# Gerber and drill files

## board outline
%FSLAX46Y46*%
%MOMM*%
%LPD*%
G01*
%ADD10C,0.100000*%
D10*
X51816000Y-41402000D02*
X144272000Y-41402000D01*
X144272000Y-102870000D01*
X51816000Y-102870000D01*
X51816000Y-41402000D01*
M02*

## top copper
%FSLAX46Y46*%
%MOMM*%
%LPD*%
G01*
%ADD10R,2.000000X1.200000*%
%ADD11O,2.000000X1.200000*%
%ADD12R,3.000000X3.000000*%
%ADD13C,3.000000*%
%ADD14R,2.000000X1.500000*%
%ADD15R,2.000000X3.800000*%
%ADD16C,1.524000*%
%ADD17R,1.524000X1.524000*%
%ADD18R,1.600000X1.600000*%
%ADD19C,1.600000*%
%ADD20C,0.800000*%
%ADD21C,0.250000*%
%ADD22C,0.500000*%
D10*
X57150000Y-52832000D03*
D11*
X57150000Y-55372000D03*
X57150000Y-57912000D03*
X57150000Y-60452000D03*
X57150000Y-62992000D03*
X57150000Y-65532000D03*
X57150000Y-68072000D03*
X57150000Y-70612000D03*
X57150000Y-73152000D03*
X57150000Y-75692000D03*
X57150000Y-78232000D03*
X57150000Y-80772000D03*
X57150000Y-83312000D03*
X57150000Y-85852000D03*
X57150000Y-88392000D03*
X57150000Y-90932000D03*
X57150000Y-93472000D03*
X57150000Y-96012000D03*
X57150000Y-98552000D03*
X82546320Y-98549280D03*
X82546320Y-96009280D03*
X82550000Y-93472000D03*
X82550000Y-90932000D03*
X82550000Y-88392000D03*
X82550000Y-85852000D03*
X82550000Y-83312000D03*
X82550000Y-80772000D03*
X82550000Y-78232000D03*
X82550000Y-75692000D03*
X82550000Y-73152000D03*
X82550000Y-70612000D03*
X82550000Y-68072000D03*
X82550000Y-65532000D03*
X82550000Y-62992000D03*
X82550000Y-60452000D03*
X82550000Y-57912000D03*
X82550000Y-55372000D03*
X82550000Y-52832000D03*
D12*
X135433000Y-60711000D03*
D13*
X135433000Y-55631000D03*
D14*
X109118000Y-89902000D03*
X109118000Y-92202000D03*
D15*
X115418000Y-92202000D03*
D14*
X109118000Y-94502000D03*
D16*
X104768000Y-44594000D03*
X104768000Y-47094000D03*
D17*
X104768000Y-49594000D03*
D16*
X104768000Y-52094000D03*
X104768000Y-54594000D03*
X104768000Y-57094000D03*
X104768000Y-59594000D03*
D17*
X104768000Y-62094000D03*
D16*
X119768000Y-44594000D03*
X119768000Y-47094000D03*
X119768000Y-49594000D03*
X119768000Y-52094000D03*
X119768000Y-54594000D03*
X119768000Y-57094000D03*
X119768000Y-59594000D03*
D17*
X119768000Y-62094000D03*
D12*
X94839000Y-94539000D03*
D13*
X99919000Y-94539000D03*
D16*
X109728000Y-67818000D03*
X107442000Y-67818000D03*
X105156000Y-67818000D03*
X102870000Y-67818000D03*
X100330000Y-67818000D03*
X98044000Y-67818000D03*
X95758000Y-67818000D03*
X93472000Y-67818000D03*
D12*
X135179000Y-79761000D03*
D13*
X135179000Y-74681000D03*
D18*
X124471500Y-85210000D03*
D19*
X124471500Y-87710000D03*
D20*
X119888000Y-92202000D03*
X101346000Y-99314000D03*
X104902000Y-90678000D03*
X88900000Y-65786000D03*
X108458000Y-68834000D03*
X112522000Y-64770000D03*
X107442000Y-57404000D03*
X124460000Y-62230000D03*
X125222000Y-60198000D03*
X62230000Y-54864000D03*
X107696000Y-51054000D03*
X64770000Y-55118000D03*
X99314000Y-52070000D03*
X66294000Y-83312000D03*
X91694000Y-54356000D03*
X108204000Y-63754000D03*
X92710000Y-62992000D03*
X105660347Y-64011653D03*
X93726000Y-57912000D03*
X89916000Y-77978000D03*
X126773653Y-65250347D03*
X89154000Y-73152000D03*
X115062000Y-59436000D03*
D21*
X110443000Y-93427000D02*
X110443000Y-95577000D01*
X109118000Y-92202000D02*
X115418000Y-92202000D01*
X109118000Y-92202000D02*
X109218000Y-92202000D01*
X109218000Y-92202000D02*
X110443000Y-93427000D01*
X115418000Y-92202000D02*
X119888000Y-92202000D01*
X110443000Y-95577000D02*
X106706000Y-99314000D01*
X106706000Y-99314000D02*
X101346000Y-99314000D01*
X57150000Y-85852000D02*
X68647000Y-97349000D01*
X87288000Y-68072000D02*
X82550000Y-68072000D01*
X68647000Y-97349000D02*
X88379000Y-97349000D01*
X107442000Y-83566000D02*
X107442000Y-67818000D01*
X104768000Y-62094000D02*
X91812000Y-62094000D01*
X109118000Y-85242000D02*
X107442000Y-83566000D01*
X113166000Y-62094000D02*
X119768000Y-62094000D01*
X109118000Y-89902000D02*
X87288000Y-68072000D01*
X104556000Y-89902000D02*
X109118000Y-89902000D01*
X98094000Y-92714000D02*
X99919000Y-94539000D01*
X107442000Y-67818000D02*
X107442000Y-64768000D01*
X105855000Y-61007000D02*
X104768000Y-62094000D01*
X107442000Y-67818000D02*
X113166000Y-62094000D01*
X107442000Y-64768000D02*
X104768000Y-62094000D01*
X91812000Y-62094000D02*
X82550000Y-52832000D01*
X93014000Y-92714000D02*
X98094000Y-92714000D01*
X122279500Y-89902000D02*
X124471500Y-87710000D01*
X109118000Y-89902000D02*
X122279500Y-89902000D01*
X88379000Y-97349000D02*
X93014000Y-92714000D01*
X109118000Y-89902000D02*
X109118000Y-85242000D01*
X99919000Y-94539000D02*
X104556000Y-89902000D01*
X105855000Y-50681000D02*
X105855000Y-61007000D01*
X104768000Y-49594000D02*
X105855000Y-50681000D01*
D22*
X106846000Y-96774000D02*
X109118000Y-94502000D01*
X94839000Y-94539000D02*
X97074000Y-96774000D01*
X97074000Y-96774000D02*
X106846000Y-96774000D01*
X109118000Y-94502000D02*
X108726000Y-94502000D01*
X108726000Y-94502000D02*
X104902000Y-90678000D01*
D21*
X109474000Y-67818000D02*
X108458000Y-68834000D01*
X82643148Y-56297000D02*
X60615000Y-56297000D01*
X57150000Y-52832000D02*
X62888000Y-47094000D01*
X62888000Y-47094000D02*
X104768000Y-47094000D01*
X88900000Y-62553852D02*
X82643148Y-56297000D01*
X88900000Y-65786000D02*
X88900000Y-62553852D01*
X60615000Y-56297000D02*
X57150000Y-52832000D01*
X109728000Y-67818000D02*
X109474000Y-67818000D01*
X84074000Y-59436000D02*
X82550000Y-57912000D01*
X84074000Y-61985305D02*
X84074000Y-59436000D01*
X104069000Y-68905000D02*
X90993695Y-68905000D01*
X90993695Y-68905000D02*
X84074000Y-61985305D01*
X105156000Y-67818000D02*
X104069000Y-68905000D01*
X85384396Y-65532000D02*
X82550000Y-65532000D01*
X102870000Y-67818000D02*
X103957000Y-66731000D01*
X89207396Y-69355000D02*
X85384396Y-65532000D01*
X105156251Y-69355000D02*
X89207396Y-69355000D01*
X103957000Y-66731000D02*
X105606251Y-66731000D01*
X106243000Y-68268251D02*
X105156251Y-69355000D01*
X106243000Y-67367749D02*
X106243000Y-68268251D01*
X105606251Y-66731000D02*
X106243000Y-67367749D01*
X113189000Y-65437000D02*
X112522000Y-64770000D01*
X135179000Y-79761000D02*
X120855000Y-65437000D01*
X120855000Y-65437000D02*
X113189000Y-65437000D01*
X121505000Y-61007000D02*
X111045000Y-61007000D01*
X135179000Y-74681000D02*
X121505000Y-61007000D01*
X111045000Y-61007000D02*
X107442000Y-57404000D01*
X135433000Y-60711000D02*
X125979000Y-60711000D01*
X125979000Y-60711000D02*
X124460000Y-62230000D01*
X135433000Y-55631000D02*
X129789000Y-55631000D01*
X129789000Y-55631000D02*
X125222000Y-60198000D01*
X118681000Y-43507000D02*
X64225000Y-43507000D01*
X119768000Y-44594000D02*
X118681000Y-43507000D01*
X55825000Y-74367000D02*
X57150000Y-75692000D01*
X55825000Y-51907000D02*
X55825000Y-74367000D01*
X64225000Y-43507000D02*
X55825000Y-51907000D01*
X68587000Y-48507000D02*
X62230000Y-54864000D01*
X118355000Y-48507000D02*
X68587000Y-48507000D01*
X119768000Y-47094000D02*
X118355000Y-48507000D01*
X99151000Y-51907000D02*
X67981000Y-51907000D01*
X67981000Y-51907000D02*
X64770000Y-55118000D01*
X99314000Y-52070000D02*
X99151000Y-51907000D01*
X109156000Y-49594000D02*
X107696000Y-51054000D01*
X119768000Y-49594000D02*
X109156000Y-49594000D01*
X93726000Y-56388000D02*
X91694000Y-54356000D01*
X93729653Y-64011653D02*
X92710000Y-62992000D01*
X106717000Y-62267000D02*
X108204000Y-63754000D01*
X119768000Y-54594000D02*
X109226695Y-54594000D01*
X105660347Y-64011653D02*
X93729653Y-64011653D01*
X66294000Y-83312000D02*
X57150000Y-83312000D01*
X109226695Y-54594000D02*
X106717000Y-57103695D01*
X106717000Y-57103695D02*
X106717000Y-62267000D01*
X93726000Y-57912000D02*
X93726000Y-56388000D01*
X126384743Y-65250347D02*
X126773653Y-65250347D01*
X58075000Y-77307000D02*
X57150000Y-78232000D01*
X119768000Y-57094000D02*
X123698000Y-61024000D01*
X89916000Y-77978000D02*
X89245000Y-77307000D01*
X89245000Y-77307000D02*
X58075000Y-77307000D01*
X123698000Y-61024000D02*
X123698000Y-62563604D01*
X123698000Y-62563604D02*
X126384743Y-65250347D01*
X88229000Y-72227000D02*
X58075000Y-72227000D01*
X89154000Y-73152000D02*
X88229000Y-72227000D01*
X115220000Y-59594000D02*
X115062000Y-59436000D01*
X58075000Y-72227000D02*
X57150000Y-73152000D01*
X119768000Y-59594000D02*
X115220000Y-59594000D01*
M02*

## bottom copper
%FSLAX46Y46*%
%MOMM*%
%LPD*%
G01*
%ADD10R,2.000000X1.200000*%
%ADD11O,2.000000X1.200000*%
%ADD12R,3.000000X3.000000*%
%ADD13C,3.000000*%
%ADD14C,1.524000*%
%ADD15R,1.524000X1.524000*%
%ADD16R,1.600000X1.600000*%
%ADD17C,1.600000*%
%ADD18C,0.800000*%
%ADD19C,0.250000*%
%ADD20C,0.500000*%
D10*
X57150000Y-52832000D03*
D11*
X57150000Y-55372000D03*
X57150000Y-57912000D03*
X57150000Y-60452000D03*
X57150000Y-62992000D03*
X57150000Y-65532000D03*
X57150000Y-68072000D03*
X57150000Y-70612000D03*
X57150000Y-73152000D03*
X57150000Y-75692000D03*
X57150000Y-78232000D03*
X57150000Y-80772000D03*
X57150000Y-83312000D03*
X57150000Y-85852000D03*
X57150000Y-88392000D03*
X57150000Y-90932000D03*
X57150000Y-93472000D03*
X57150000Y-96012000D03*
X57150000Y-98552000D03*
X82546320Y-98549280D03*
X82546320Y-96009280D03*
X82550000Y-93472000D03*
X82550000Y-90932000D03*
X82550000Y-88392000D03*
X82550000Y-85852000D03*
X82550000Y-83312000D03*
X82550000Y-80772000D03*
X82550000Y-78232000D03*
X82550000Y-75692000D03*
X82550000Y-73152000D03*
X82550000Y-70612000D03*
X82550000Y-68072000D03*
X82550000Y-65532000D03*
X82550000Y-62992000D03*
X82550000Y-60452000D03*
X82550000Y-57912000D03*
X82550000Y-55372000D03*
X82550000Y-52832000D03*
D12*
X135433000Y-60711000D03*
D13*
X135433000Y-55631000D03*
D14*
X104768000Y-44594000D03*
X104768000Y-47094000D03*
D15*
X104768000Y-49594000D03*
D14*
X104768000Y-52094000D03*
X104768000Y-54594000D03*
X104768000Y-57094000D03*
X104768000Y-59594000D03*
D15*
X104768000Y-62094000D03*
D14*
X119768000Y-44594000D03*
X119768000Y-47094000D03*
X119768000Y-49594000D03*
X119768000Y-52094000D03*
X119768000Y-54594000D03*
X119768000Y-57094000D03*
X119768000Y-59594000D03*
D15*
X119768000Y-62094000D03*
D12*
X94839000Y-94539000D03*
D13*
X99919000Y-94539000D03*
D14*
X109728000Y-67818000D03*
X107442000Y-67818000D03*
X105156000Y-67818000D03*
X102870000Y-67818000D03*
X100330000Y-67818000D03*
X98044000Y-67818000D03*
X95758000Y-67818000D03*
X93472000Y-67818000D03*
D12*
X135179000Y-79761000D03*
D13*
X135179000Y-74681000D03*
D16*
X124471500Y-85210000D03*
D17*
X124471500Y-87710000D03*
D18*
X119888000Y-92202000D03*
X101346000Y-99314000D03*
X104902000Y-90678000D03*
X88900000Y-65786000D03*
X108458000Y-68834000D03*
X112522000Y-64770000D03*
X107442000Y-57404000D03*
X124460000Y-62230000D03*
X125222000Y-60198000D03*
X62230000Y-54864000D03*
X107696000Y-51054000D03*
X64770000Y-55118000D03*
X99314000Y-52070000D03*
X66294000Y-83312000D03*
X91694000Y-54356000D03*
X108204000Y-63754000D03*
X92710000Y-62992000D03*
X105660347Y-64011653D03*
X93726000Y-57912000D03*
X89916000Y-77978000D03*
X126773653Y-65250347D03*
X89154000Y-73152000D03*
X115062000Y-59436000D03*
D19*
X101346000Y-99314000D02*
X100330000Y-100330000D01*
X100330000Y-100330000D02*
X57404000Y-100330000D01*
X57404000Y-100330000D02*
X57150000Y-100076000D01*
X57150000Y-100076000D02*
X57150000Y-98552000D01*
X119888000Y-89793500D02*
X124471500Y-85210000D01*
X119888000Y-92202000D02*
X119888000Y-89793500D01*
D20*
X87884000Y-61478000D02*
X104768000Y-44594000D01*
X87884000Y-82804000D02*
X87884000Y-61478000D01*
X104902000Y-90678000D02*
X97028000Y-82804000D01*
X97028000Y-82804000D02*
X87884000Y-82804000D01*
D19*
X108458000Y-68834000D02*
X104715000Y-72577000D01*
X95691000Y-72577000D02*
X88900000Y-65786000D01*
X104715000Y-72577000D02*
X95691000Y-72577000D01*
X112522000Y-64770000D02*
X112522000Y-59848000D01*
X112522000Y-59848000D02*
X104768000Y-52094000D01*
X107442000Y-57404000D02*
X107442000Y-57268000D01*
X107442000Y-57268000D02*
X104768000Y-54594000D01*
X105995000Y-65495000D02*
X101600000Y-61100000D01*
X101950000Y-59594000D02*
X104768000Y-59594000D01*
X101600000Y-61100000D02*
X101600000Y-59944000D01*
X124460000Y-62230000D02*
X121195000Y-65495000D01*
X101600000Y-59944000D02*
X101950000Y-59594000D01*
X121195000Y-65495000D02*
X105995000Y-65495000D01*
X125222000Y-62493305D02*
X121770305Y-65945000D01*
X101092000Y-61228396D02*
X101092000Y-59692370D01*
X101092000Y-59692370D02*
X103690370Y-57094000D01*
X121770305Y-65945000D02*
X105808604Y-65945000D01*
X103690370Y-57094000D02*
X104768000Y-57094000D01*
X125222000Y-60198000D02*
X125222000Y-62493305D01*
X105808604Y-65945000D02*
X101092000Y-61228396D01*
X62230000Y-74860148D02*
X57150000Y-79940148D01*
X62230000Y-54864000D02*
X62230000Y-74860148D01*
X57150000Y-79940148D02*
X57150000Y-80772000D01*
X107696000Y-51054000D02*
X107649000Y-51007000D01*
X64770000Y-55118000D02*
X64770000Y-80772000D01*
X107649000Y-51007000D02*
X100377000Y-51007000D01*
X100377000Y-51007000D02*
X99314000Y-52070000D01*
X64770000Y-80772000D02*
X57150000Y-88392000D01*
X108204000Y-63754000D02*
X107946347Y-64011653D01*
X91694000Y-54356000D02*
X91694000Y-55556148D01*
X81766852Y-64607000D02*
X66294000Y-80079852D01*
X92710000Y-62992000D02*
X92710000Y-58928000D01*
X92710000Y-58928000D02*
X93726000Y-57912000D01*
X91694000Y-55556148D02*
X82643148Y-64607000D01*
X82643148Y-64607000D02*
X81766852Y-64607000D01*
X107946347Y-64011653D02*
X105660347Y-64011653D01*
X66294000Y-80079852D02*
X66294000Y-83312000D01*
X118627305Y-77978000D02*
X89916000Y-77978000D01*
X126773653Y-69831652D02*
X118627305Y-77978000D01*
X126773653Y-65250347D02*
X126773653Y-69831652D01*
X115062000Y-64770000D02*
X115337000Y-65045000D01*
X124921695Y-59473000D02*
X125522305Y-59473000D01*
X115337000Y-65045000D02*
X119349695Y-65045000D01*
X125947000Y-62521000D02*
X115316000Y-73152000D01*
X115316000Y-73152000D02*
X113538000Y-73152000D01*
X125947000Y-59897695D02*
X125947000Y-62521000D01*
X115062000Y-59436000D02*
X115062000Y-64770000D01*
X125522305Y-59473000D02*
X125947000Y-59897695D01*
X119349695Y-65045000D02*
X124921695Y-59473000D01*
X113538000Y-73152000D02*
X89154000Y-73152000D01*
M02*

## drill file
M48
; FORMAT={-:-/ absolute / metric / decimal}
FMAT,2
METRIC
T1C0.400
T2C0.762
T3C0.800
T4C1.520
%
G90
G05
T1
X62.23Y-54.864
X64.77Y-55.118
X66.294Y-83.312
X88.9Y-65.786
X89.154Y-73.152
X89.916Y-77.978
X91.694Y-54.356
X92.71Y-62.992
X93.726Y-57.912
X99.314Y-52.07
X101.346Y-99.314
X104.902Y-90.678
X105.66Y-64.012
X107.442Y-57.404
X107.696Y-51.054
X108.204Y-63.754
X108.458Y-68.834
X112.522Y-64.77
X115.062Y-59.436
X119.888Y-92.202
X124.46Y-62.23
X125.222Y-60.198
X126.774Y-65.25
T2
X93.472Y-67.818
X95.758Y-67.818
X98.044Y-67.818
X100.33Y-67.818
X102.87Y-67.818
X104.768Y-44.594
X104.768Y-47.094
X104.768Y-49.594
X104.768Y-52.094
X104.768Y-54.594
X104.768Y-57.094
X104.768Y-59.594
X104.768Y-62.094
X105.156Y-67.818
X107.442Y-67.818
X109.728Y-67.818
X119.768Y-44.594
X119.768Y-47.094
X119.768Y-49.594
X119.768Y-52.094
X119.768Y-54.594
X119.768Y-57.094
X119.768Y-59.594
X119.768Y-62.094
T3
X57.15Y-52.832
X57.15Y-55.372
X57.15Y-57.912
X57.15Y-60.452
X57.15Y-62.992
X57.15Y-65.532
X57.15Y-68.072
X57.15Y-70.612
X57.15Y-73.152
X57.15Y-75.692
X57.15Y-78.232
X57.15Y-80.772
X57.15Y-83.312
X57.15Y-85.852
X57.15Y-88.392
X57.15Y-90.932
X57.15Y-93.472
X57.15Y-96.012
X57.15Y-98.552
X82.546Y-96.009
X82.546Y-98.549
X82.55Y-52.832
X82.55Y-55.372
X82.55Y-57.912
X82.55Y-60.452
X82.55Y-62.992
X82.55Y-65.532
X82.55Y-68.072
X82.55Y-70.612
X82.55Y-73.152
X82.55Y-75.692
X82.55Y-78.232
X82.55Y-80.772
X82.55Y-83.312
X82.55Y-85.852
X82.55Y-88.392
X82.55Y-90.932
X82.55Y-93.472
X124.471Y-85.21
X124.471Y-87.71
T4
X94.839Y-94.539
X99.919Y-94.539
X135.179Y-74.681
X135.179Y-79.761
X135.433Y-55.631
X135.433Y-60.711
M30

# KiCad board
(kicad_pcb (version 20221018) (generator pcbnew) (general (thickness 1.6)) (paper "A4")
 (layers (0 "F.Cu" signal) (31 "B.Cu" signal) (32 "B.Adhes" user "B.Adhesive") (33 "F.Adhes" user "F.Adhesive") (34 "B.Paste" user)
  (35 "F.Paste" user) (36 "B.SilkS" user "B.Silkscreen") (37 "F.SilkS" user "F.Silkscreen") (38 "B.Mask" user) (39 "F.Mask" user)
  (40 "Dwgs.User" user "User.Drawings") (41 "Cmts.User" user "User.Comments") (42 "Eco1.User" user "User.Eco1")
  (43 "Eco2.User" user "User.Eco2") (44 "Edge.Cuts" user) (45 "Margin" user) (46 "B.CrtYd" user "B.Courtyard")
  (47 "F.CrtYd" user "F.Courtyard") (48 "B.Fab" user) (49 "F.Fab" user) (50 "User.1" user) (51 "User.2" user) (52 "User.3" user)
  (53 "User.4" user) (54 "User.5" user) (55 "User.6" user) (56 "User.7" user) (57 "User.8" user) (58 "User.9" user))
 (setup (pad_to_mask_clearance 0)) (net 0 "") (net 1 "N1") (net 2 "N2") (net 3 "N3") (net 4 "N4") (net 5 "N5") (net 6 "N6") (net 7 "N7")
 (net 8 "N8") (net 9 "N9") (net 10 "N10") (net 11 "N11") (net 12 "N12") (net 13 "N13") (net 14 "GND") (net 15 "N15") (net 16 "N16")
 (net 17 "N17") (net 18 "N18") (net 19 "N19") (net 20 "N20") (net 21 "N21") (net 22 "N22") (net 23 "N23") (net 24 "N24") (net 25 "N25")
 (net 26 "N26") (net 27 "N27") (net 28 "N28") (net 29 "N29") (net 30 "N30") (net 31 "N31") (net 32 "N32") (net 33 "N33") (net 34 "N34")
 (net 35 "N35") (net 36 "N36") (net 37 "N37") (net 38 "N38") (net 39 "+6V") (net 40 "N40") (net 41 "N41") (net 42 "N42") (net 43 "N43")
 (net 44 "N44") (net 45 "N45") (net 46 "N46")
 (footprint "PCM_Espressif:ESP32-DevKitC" (layer "F.Cu") (at 57.15 52.832)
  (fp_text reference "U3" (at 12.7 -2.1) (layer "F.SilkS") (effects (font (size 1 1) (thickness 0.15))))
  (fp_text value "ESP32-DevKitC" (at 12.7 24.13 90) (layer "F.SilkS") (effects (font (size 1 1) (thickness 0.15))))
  (pad "1" thru_hole rect (at 0 0 270) (size 1.2 2) (drill 0.8) (layers "*.Cu" "*.Mask") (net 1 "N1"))
  (pad "2" thru_hole oval (at 0 2.54 270) (size 1.2 2) (drill 0.8) (layers "*.Cu" "*.Mask") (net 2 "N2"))
  (pad "3" thru_hole oval (at 0 5.08 270) (size 1.2 2) (drill 0.8) (layers "*.Cu" "*.Mask") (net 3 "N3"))
  (pad "4" thru_hole oval (at 0 7.62 270) (size 1.2 2) (drill 0.8) (layers "*.Cu" "*.Mask") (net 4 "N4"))
  (pad "5" thru_hole oval (at 0 10.16 270) (size 1.2 2) (drill 0.8) (layers "*.Cu" "*.Mask") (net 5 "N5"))
  (pad "6" thru_hole oval (at 0 12.7 270) (size 1.2 2) (drill 0.8) (layers "*.Cu" "*.Mask") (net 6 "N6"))
  (pad "7" thru_hole oval (at 0 15.24 270) (size 1.2 2) (drill 0.8) (layers "*.Cu" "*.Mask") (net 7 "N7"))
  (pad "8" thru_hole oval (at 0 17.78 270) (size 1.2 2) (drill 0.8) (layers "*.Cu" "*.Mask") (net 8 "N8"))
  (pad "9" thru_hole oval (at 0 20.32 270) (size 1.2 2) (drill 0.8) (layers "*.Cu" "*.Mask") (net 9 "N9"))
  (pad "10" thru_hole oval (at 0 22.86 270) (size 1.2 2) (drill 0.8) (layers "*.Cu" "*.Mask") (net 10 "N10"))
  (pad "11" thru_hole oval (at 0 25.4 270) (size 1.2 2) (drill 0.8) (layers "*.Cu" "*.Mask") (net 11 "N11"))
  (pad "12" thru_hole oval (at 0 27.94 270) (size 1.2 2) (drill 0.8) (layers "*.Cu" "*.Mask") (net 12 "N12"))
  (pad "13" thru_hole oval (at 0 30.48 270) (size 1.2 2) (drill 0.8) (layers "*.Cu" "*.Mask") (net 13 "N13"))
  (pad "14" thru_hole oval (at 0 33.02 270) (size 1.2 2) (drill 0.8) (layers "*.Cu" "*.Mask") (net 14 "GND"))
  (pad "15" thru_hole oval (at 0 35.56 270) (size 1.2 2) (drill 0.8) (layers "*.Cu" "*.Mask") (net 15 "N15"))
  (pad "16" thru_hole oval (at 0 38.1 270) (size 1.2 2) (drill 0.8) (layers "*.Cu" "*.Mask") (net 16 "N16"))
  (pad "17" thru_hole oval (at 0 40.64 270) (size 1.2 2) (drill 0.8) (layers "*.Cu" "*.Mask") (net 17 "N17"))
  (pad "18" thru_hole oval (at 0 43.18 270) (size 1.2 2) (drill 0.8) (layers "*.Cu" "*.Mask") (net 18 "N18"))
  (pad "19" thru_hole oval (at 0 45.72 270) (size 1.2 2) (drill 0.8) (layers "*.Cu" "*.Mask") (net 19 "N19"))
  (pad "20" thru_hole oval (at 25.39632 45.71728 270) (size 1.2 2) (drill 0.8) (layers "*.Cu" "*.Mask") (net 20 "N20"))
  (pad "21" thru_hole oval (at 25.39632 43.17728 270) (size 1.2 2) (drill 0.8) (layers "*.Cu" "*.Mask") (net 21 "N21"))
  (pad "22" thru_hole oval (at 25.4 40.64 270) (size 1.2 2) (drill 0.8) (layers "*.Cu" "*.Mask") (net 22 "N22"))
  (pad "23" thru_hole oval (at 25.4 38.1 270) (size 1.2 2) (drill 0.8) (layers "*.Cu" "*.Mask") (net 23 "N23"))
  (pad "24" thru_hole oval (at 25.4 35.56 270) (size 1.2 2) (drill 0.8) (layers "*.Cu" "*.Mask") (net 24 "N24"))
  (pad "25" thru_hole oval (at 25.4 33.02 270) (size 1.2 2) (drill 0.8) (layers "*.Cu" "*.Mask") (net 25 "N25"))
  (pad "26" thru_hole oval (at 25.4 30.48 270) (size 1.2 2) (drill 0.8) (layers "*.Cu" "*.Mask") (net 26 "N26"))
  (pad "27" thru_hole oval (at 25.4 27.94 270) (size 1.2 2) (drill 0.8) (layers "*.Cu" "*.Mask") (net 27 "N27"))
  (pad "28" thru_hole oval (at 25.4 25.4 270) (size 1.2 2) (drill 0.8) (layers "*.Cu" "*.Mask") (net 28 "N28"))
  (pad "29" thru_hole oval (at 25.4 22.86 270) (size 1.2 2) (drill 0.8) (layers "*.Cu" "*.Mask") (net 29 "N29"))
  (pad "30" thru_hole oval (at 25.4 20.32 270) (size 1.2 2) (drill 0.8) (layers "*.Cu" "*.Mask") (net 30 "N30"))
  (pad "31" thru_hole oval (at 25.4 17.78 270) (size 1.2 2) (drill 0.8) (layers "*.Cu" "*.Mask") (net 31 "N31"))
  (pad "32" thru_hole oval (at 25.4 15.24 270) (size 1.2 2) (drill 0.8) (layers "*.Cu" "*.Mask") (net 14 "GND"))
  (pad "33" thru_hole oval (at 25.4 12.7 270) (size 1.2 2) (drill 0.8) (layers "*.Cu" "*.Mask") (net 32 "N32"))
  (pad "34" thru_hole oval (at 25.4 10.16 270) (size 1.2 2) (drill 0.8) (layers "*.Cu" "*.Mask") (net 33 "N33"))
  (pad "35" thru_hole oval (at 25.4 7.62 270) (size 1.2 2) (drill 0.8) (layers "*.Cu" "*.Mask") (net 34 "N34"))
  (pad "36" thru_hole oval (at 25.4 5.08 270) (size 1.2 2) (drill 0.8) (layers "*.Cu" "*.Mask") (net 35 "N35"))
  (pad "37" thru_hole oval (at 25.4 2.54 270) (size 1.2 2) (drill 0.8) (layers "*.Cu" "*.Mask") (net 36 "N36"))
  (pad "38" thru_hole oval (at 25.4 0 270) (size 1.2 2) (drill 0.8) (layers "*.Cu" "*.Mask") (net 14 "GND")))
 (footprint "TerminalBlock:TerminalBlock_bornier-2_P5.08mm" (layer "F.Cu") (at 135.433 60.711 90)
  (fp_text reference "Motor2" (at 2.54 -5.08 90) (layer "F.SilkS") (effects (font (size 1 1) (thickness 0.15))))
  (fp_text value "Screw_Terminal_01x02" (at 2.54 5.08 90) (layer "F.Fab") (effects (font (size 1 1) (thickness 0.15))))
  (pad "1" thru_hole rect (at 0 0 90) (size 3 3) (drill 1.52) (layers "*.Cu" "*.Mask") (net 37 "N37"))
  (pad "2" thru_hole circle (at 5.08 0 90) (size 3 3) (drill 1.52) (layers "*.Cu" "*.Mask") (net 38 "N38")))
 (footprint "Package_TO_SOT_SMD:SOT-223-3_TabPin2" (layer "F.Cu") (at 112.268 92.202)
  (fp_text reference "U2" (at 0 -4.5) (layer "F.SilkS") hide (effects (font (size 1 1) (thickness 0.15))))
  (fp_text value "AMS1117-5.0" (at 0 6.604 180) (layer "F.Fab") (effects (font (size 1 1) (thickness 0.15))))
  (pad "1" smd rect (at -3.15 -2.3) (size 2 1.5) (layers "F.Cu" "F.Paste" "F.Mask") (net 14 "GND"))
  (pad "2" smd rect (at -3.15 0) (size 2 1.5) (layers "F.Cu" "F.Paste" "F.Mask") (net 19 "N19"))
  (pad "2" smd rect (at 3.15 0) (size 2 3.8) (layers "F.Cu" "F.Paste" "F.Mask") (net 19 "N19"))
  (pad "3" smd rect (at -3.15 2.3) (size 2 1.5) (layers "F.Cu" "F.Paste" "F.Mask") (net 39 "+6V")))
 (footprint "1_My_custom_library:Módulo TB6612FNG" (layer "F.Cu") (at 112.268 53.594)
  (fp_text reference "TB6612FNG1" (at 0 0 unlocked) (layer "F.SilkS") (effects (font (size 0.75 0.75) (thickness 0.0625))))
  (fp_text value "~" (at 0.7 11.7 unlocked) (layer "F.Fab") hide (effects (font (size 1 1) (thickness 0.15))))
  (pad "1" thru_hole circle (at -7.5 -9) (size 1.524 1.524) (drill 0.762) (layers "*.Cu" "*.Mask") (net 39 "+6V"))
  (pad "2" thru_hole circle (at -7.5 -6.5) (size 1.524 1.524) (drill 0.762) (layers "*.Cu" "*.Mask") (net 1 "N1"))
  (pad "3" thru_hole rect (at -7.5 -4) (size 1.524 1.524) (drill 0.762) (layers "*.Cu" "*.Mask") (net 14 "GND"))
  (pad "4" thru_hole circle (at -7.5 -1.5) (size 1.524 1.524) (drill 0.762) (layers "*.Cu" "*.Mask") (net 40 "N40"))
  (pad "5" thru_hole circle (at -7.5 1) (size 1.524 1.524) (drill 0.762) (layers "*.Cu" "*.Mask") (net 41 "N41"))
  (pad "6" thru_hole circle (at -7.5 3.5) (size 1.524 1.524) (drill 0.762) (layers "*.Cu" "*.Mask") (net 38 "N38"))
  (pad "7" thru_hole circle (at -7.5 6) (size 1.524 1.524) (drill 0.762) (layers "*.Cu" "*.Mask") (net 37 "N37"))
  (pad "8" thru_hole rect (at -7.5 8.5) (size 1.524 1.524) (drill 0.762) (layers "*.Cu" "*.Mask") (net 14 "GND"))
  (pad "9" thru_hole circle (at 7.5 -9) (size 1.524 1.524) (drill 0.762) (layers "*.Cu" "*.Mask") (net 10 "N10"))
  (pad "10" thru_hole circle (at 7.5 -6.5) (size 1.524 1.524) (drill 0.762) (layers "*.Cu" "*.Mask") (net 12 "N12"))
  (pad "11" thru_hole circle (at 7.5 -4) (size 1.524 1.524) (drill 0.762) (layers "*.Cu" "*.Mask") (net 15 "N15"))
  (pad "12" thru_hole circle (at 7.5 -1.5) (size 1.524 1.524) (drill 0.762) (layers "*.Cu" "*.Mask") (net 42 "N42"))
  (pad "13" thru_hole circle (at 7.5 1) (size 1.524 1.524) (drill 0.762) (layers "*.Cu" "*.Mask") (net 13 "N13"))
  (pad "14" thru_hole circle (at 7.5 3.5) (size 1.524 1.524) (drill 0.762) (layers "*.Cu" "*.Mask") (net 11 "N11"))
  (pad "15" thru_hole circle (at 7.5 6) (size 1.524 1.524) (drill 0.762) (layers "*.Cu" "*.Mask") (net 9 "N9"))
  (pad "16" thru_hole rect (at 7.5 8.5) (size 1.524 1.524) (drill 0.762) (layers "*.Cu" "*.Mask") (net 14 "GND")))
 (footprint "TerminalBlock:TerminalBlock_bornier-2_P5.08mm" (layer "F.Cu") (at 94.839 94.539)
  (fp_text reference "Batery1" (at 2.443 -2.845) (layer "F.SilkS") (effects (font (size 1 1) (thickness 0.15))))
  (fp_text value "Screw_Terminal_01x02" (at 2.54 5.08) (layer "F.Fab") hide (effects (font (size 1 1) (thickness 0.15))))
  (pad "1" thru_hole rect (at 0 0) (size 3 3) (drill 1.52) (layers "*.Cu" "*.Mask") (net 39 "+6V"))
  (pad "2" thru_hole circle (at 5.08 0) (size 3 3) (drill 1.52) (layers "*.Cu" "*.Mask") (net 14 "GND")))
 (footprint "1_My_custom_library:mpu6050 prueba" (layer "F.Cu") (at 101.346 73.406 -90)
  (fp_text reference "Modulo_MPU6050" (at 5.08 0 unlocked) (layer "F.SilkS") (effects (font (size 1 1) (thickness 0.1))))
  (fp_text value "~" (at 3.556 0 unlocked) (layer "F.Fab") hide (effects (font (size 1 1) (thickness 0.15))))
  (pad "1" thru_hole circle (at -5.588 -8.382 270) (size 1.524 1.524) (drill 0.762) (layers "*.Cu" "*.Mask") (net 1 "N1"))
  (pad "2" thru_hole circle (at -5.588 -6.096 270) (size 1.524 1.524) (drill 0.762) (layers "*.Cu" "*.Mask") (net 14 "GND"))
  (pad "3" thru_hole circle (at -5.588 -3.81 270) (size 1.524 1.524) (drill 0.762) (layers "*.Cu" "*.Mask") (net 35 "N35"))
  (pad "4" thru_hole circle (at -5.588 -1.524 270) (size 1.524 1.524) (drill 0.762) (layers "*.Cu" "*.Mask") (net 32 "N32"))
  (pad "5" thru_hole circle (at -5.588 1.016 270) (size 1.524 1.524) (drill 0.762) (layers "*.Cu" "*.Mask") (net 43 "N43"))
  (pad "6" thru_hole circle (at -5.588 3.302 270) (size 1.524 1.524) (drill 0.762) (layers "*.Cu" "*.Mask") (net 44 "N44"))
  (pad "7" thru_hole circle (at -5.588 5.588 270) (size 1.524 1.524) (drill 0.762) (layers "*.Cu" "*.Mask") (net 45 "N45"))
  (pad "8" thru_hole circle (at -5.588 7.874 270) (size 1.524 1.524) (drill 0.762) (layers "*.Cu" "*.Mask") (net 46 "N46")))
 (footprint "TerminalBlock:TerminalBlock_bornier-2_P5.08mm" (layer "F.Cu") (at 135.179 79.761 90)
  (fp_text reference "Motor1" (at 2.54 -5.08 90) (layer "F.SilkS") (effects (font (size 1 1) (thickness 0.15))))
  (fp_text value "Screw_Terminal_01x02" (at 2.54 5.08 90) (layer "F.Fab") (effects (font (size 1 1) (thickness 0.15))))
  (pad "1" thru_hole rect (at 0 0 90) (size 3 3) (drill 1.52) (layers "*.Cu" "*.Mask") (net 40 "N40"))
  (pad "2" thru_hole circle (at 5.08 0 90) (size 3 3) (drill 1.52) (layers "*.Cu" "*.Mask") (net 41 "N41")))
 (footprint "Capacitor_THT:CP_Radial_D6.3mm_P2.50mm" (layer "F.Cu") (at 124.4715 85.21 -90)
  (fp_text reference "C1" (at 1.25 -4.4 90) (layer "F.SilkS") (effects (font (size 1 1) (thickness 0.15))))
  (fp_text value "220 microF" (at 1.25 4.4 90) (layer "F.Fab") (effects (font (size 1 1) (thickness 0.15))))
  (pad "1" thru_hole rect (at 0 0 270) (size 1.6 1.6) (drill 0.8) (layers "*.Cu" "*.Mask") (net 19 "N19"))
  (pad "2" thru_hole circle (at 2.5 0 270) (size 1.6 1.6) (drill 0.8) (layers "*.Cu" "*.Mask") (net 14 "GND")))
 (gr_rect (start 51.816 41.402) (end 144.272 102.87) (stroke (width 0.1) (type default)) (fill none) (layer "Edge.Cuts"))
 (segment (start 110.443 93.427) (end 110.443 95.577) (width 0.25) (layer "F.Cu") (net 19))
 (segment (start 109.118 92.202) (end 115.418 92.202) (width 0.25) (layer "F.Cu") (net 19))
 (segment (start 109.118 92.202) (end 109.218 92.202) (width 0.25) (layer "F.Cu") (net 19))
 (segment (start 109.218 92.202) (end 110.443 93.427) (width 0.25) (layer "F.Cu") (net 19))
 (segment (start 115.418 92.202) (end 119.888 92.202) (width 0.25) (layer "F.Cu") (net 19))
 (segment (start 110.443 95.577) (end 106.706 99.314) (width 0.25) (layer "F.Cu") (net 19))
 (segment (start 106.706 99.314) (end 101.346 99.314) (width 0.25) (layer "F.Cu") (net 19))
 (via (at 119.888 92.202) (size 0.8) (drill 0.4) (layers "F.Cu" "B.Cu") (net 19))
 (via (at 101.346 99.314) (size 0.8) (drill 0.4) (layers "F.Cu" "B.Cu") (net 19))
 (segment (start 101.346 99.314) (end 100.33 100.33) (width 0.25) (layer "B.Cu") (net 19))
 (segment (start 100.33 100.33) (end 57.404 100.33) (width 0.25) (layer "B.Cu") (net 19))
 (segment (start 57.404 100.33) (end 57.15 100.076) (width 0.25) (layer "B.Cu") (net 19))
 (segment (start 57.15 100.076) (end 57.15 98.552) (width 0.25) (layer "B.Cu") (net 19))
 (segment (start 119.888 89.7935) (end 124.4715 85.21) (width 0.25) (layer "B.Cu") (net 19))
 (segment (start 119.888 92.202) (end 119.888 89.7935) (width 0.25) (layer "B.Cu") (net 19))
 (segment (start 57.15 85.852) (end 68.647 97.349) (width 0.25) (layer "F.Cu") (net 14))
 (segment (start 87.288 68.072) (end 82.55 68.072) (width 0.25) (layer "F.Cu") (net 14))
 (segment (start 68.647 97.349) (end 88.379 97.349) (width 0.25) (layer "F.Cu") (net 14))
 (segment (start 107.442 83.566) (end 107.442 67.818) (width 0.25) (layer "F.Cu") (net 14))
 (segment (start 104.768 62.094) (end 91.812 62.094) (width 0.25) (layer "F.Cu") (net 14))
 (segment (start 109.118 85.242) (end 107.442 83.566) (width 0.25) (layer "F.Cu") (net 14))
 (segment (start 113.166 62.094) (end 119.768 62.094) (width 0.25) (layer "F.Cu") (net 14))
 (segment (start 109.118 89.902) (end 87.288 68.072) (width 0.25) (layer "F.Cu") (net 14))
 (segment (start 104.556 89.902) (end 109.118 89.902) (width 0.25) (layer "F.Cu") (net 14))
 (segment (start 98.094 92.714) (end 99.919 94.539) (width 0.25) (layer "F.Cu") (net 14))
 (segment (start 107.442 67.818) (end 107.442 64.768) (width 0.25) (layer "F.Cu") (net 14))
 (segment (start 105.855 61.007) (end 104.768 62.094) (width 0.25) (layer "F.Cu") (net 14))
 (segment (start 107.442 67.818) (end 113.166 62.094) (width 0.25) (layer "F.Cu") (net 14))
 (segment (start 107.442 64.768) (end 104.768 62.094) (width 0.25) (layer "F.Cu") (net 14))
 (segment (start 91.812 62.094) (end 82.55 52.832) (width 0.25) (layer "F.Cu") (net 14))
 (segment (start 93.014 92.714) (end 98.094 92.714) (width 0.25) (layer "F.Cu") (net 14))
 (segment (start 122.2795 89.902) (end 124.4715 87.71) (width 0.25) (layer "F.Cu") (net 14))
 (segment (start 109.118 89.902) (end 122.2795 89.902) (width 0.25) (layer "F.Cu") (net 14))
 (segment (start 88.379 97.349) (end 93.014 92.714) (width 0.25) (layer "F.Cu") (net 14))
 (segment (start 109.118 89.902) (end 109.118 85.242) (width 0.25) (layer "F.Cu") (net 14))
 (segment (start 99.919 94.539) (end 104.556 89.902) (width 0.25) (layer "F.Cu") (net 14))
 (segment (start 105.855 50.681) (end 105.855 61.007) (width 0.25) (layer "F.Cu") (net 14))
 (segment (start 104.768 49.594) (end 105.855 50.681) (width 0.25) (layer "F.Cu") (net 14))
 (segment (start 106.846 96.774) (end 109.118 94.502) (width 0.5) (layer "F.Cu") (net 39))
 (segment (start 94.839 94.539) (end 97.074 96.774) (width 0.5) (layer "F.Cu") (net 39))
 (segment (start 97.074 96.774) (end 106.846 96.774) (width 0.5) (layer "F.Cu") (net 39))
 (segment (start 109.118 94.502) (end 108.726 94.502) (width 0.5) (layer "F.Cu") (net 39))
 (segment (start 108.726 94.502) (end 104.902 90.678) (width 0.5) (layer "F.Cu") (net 39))
 (via (at 104.902 90.678) (size 0.8) (drill 0.4) (layers "F.Cu" "B.Cu") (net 39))
 (segment (start 87.884 61.478) (end 104.768 44.594) (width 0.5) (layer "B.Cu") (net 39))
 (segment (start 87.884 82.804) (end 87.884 61.478) (width 0.5) (layer "B.Cu") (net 39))
 (segment (start 104.902 90.678) (end 97.028 82.804) (width 0.5) (layer "B.Cu") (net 39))
 (segment (start 97.028 82.804) (end 87.884 82.804) (width 0.5) (layer "B.Cu") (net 39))
 (segment (start 109.474 67.818) (end 108.458 68.834) (width 0.25) (layer "F.Cu") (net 1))
 (segment (start 82.643148 56.297) (end 60.615 56.297) (width 0.25) (layer "F.Cu") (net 1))
 (segment (start 57.15 52.832) (end 62.888 47.094) (width 0.25) (layer "F.Cu") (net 1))
 (segment (start 62.888 47.094) (end 104.768 47.094) (width 0.25) (layer "F.Cu") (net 1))
 (segment (start 88.9 62.553852) (end 82.643148 56.297) (width 0.25) (layer "F.Cu") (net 1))
 (segment (start 88.9 65.786) (end 88.9 62.553852) (width 0.25) (layer "F.Cu") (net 1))
 (segment (start 60.615 56.297) (end 57.15 52.832) (width 0.25) (layer "F.Cu") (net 1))
 (segment (start 109.728 67.818) (end 109.474 67.818) (width 0.25) (layer "F.Cu") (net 1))
 (via (at 88.9 65.786) (size 0.8) (drill 0.4) (layers "F.Cu" "B.Cu") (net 1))
 (via (at 108.458 68.834) (size 0.8) (drill 0.4) (layers "F.Cu" "B.Cu") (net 1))
 (segment (start 108.458 68.834) (end 104.715 72.577) (width 0.25) (layer "B.Cu") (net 1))
 (segment (start 95.691 72.577) (end 88.9 65.786) (width 0.25) (layer "B.Cu") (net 1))
 (segment (start 104.715 72.577) (end 95.691 72.577) (width 0.25) (layer "B.Cu") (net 1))
 (segment (start 84.074 59.436) (end 82.55 57.912) (width 0.25) (layer "F.Cu") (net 35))
 (segment (start 84.074 61.985305) (end 84.074 59.436) (width 0.25) (layer "F.Cu") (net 35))
 (segment (start 104.069 68.905) (end 90.993695 68.905) (width 0.25) (layer "F.Cu") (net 35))
 (segment (start 90.993695 68.905) (end 84.074 61.985305) (width 0.25) (layer "F.Cu") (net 35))
 (segment (start 105.156 67.818) (end 104.069 68.905) (width 0.25) (layer "F.Cu") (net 35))
 (segment (start 85.384396 65.532) (end 82.55 65.532) (width 0.25) (layer "F.Cu") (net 32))
 (segment (start 102.87 67.818) (end 103.957 66.731) (width 0.25) (layer "F.Cu") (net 32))
 (segment (start 89.207396 69.355) (end 85.384396 65.532) (width 0.25) (layer "F.Cu") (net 32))
 (segment (start 105.156251 69.355) (end 89.207396 69.355) (width 0.25) (layer "F.Cu") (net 32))
 (segment (start 103.957 66.731) (end 105.606251 66.731) (width 0.25) (layer "F.Cu") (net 32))
 (segment (start 106.243 68.268251) (end 105.156251 69.355) (width 0.25) (layer "F.Cu") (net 32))
 (segment (start 106.243 67.367749) (end 106.243 68.268251) (width 0.25) (layer "F.Cu") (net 32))
 (segment (start 105.606251 66.731) (end 106.243 67.367749) (width 0.25) (layer "F.Cu") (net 32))
 (segment (start 113.189 65.437) (end 112.522 64.77) (width 0.25) (layer "F.Cu") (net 40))
 (segment (start 135.179 79.761) (end 120.855 65.437) (width 0.25) (layer "F.Cu") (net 40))
 (segment (start 120.855 65.437) (end 113.189 65.437) (width 0.25) (layer "F.Cu") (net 40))
 (via (at 112.522 64.77) (size 0.8) (drill 0.4) (layers "F.Cu" "B.Cu") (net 40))
 (segment (start 112.522 64.77) (end 112.522 59.848) (width 0.25) (layer "B.Cu") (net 40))
 (segment (start 112.522 59.848) (end 104.768 52.094) (width 0.25) (layer "B.Cu") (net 40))
 (segment (start 121.505 61.007) (end 111.045 61.007) (width 0.25) (layer "F.Cu") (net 41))
 (segment (start 135.179 74.681) (end 121.505 61.007) (width 0.25) (layer "F.Cu") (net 41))
 (segment (start 111.045 61.007) (end 107.442 57.404) (width 0.25) (layer "F.Cu") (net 41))
 (via (at 107.442 57.404) (size 0.8) (drill 0.4) (layers "F.Cu" "B.Cu") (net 41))
 (segment (start 107.442 57.404) (end 107.442 57.268) (width 0.25) (layer "B.Cu") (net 41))
 (segment (start 107.442 57.268) (end 104.768 54.594) (width 0.25) (layer "B.Cu") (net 41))
 (segment (start 135.433 60.711) (end 125.979 60.711) (width 0.25) (layer "F.Cu") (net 37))
 (segment (start 125.979 60.711) (end 124.46 62.23) (width 0.25) (layer "F.Cu") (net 37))
 (via (at 124.46 62.23) (size 0.8) (drill 0.4) (layers "F.Cu" "B.Cu") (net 37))
 (segment (start 105.995 65.495) (end 101.6 61.1) (width 0.25) (layer "B.Cu") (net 37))
 (segment (start 101.95 59.594) (end 104.768 59.594) (width 0.25) (layer "B.Cu") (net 37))
 (segment (start 101.6 61.1) (end 101.6 59.944) (width 0.25) (layer "B.Cu") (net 37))
 (segment (start 124.46 62.23) (end 121.195 65.495) (width 0.25) (layer "B.Cu") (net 37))
 (segment (start 101.6 59.944) (end 101.95 59.594) (width 0.25) (layer "B.Cu") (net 37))
 (segment (start 121.195 65.495) (end 105.995 65.495) (width 0.25) (layer "B.Cu") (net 37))
 (segment (start 135.433 55.631) (end 129.789 55.631) (width 0.25) (layer "F.Cu") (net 38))
 (segment (start 129.789 55.631) (end 125.222 60.198) (width 0.25) (layer "F.Cu") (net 38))
 (via (at 125.222 60.198) (size 0.8) (drill 0.4) (layers "F.Cu" "B.Cu") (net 38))
 (segment (start 125.222 62.493305) (end 121.770305 65.945) (width 0.25) (layer "B.Cu") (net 38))
 (segment (start 101.092 61.228396) (end 101.092 59.69237) (width 0.25) (layer "B.Cu") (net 38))
 (segment (start 101.092 59.69237) (end 103.69037 57.094) (width 0.25) (layer "B.Cu") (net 38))
 (segment (start 121.770305 65.945) (end 105.808604 65.945) (width 0.25) (layer "B.Cu") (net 38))
 (segment (start 103.69037 57.094) (end 104.768 57.094) (width 0.25) (layer "B.Cu") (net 38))
 (segment (start 125.222 60.198) (end 125.222 62.493305) (width 0.25) (layer "B.Cu") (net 38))
 (segment (start 105.808604 65.945) (end 101.092 61.228396) (width 0.25) (layer "B.Cu") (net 38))
 (segment (start 118.681 43.507) (end 64.225 43.507) (width 0.25) (layer "F.Cu") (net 10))
 (segment (start 119.768 44.594) (end 118.681 43.507) (width 0.25) (layer "F.Cu") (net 10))
 (segment (start 55.825 74.367) (end 57.15 75.692) (width 0.25) (layer "F.Cu") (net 10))
 (segment (start 55.825 51.907) (end 55.825 74.367) (width 0.25) (layer "F.Cu") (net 10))
 (segment (start 64.225 43.507) (end 55.825 51.907) (width 0.25) (layer "F.Cu") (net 10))
 (segment (start 68.587 48.507) (end 62.23 54.864) (width 0.25) (layer "F.Cu") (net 12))
 (segment (start 118.355 48.507) (end 68.587 48.507) (width 0.25) (layer "F.Cu") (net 12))
 (segment (start 119.768 47.094) (end 118.355 48.507) (width 0.25) (layer "F.Cu") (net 12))
 (via (at 62.23 54.864) (size 0.8) (drill 0.4) (layers "F.Cu" "B.Cu") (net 12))
 (segment (start 62.23 74.860148) (end 57.15 79.940148) (width 0.25) (layer "B.Cu") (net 12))
 (segment (start 62.23 54.864) (end 62.23 74.860148) (width 0.25) (layer "B.Cu") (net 12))
 (segment (start 57.15 79.940148) (end 57.15 80.772) (width 0.25) (layer "B.Cu") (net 12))
 (segment (start 99.151 51.907) (end 67.981 51.907) (width 0.25) (layer "F.Cu") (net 15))
 (segment (start 67.981 51.907) (end 64.77 55.118) (width 0.25) (layer "F.Cu") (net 15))
 (segment (start 99.314 52.07) (end 99.151 51.907) (width 0.25) (layer "F.Cu") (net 15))
 (segment (start 109.156 49.594) (end 107.696 51.054) (width 0.25) (layer "F.Cu") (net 15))
 (segment (start 119.768 49.594) (end 109.156 49.594) (width 0.25) (layer "F.Cu") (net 15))
 (via (at 107.696 51.054) (size 0.8) (drill 0.4) (layers "F.Cu" "B.Cu") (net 15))
 (via (at 64.77 55.118) (size 0.8) (drill 0.4) (layers "F.Cu" "B.Cu") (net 15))
 (via (at 99.314 52.07) (size 0.8) (drill 0.4) (layers "F.Cu" "B.Cu") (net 15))
 (segment (start 107.696 51.054) (end 107.649 51.007) (width 0.25) (layer "B.Cu") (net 15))
 (segment (start 64.77 55.118) (end 64.77 80.772) (width 0.25) (layer "B.Cu") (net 15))
 (segment (start 107.649 51.007) (end 100.377 51.007) (width 0.25) (layer "B.Cu") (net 15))
 (segment (start 100.377 51.007) (end 99.314 52.07) (width 0.25) (layer "B.Cu") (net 15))
 (segment (start 64.77 80.772) (end 57.15 88.392) (width 0.25) (layer "B.Cu") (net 15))
 (segment (start 93.726 56.388) (end 91.694 54.356) (width 0.25) (layer "F.Cu") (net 13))
 (segment (start 93.729653 64.011653) (end 92.71 62.992) (width 0.25) (layer "F.Cu") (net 13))
 (segment (start 106.717 62.267) (end 108.204 63.754) (width 0.25) (layer "F.Cu") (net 13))
 (segment (start 119.768 54.594) (end 109.226695 54.594) (width 0.25) (layer "F.Cu") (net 13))
 (segment (start 105.660347 64.011653) (end 93.729653 64.011653) (width 0.25) (layer "F.Cu") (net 13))
 (segment (start 66.294 83.312) (end 57.15 83.312) (width 0.25) (layer "F.Cu") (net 13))
 (segment (start 109.226695 54.594) (end 106.717 57.103695) (width 0.25) (layer "F.Cu") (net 13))
 (segment (start 106.717 57.103695) (end 106.717 62.267) (width 0.25) (layer "F.Cu") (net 13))
 (segment (start 93.726 57.912) (end 93.726 56.388) (width 0.25) (layer "F.Cu") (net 13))
 (via (at 66.294 83.312) (size 0.8) (drill 0.4) (layers "F.Cu" "B.Cu") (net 13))
 (via (at 91.694 54.356) (size 0.8) (drill 0.4) (layers "F.Cu" "B.Cu") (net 13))
 (via (at 108.204 63.754) (size 0.8) (drill 0.4) (layers "F.Cu" "B.Cu") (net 13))
 (via (at 92.71 62.992) (size 0.8) (drill 0.4) (layers "F.Cu" "B.Cu") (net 13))
 (via (at 105.660347 64.011653) (size 0.8) (drill 0.4) (layers "F.Cu" "B.Cu") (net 13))
 (via (at 93.726 57.912) (size 0.8) (drill 0.4) (layers "F.Cu" "B.Cu") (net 13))
 (segment (start 108.204 63.754) (end 107.946347 64.011653) (width 0.25) (layer "B.Cu") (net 13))
 (segment (start 91.694 54.356) (end 91.694 55.556148) (width 0.25) (layer "B.Cu") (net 13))
 (segment (start 81.766852 64.607) (end 66.294 80.079852) (width 0.25) (layer "B.Cu") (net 13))
 (segment (start 92.71 62.992) (end 92.71 58.928) (width 0.25) (layer "B.Cu") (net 13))
 (segment (start 92.71 58.928) (end 93.726 57.912) (width 0.25) (layer "B.Cu") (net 13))
 (segment (start 91.694 55.556148) (end 82.643148 64.607) (width 0.25) (layer "B.Cu") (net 13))
 (segment (start 82.643148 64.607) (end 81.766852 64.607) (width 0.25) (layer "B.Cu") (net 13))
 (segment (start 107.946347 64.011653) (end 105.660347 64.011653) (width 0.25) (layer "B.Cu") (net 13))
 (segment (start 66.294 80.079852) (end 66.294 83.312) (width 0.25) (layer "B.Cu") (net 13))
 (segment (start 126.384743 65.250347) (end 126.773653 65.250347) (width 0.25) (layer "F.Cu") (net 11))
 (segment (start 58.075 77.307) (end 57.15 78.232) (width 0.25) (layer "F.Cu") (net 11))
 (segment (start 119.768 57.094) (end 123.698 61.024) (width 0.25) (layer "F.Cu") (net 11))
 (segment (start 89.916 77.978) (end 89.245 77.307) (width 0.25) (layer "F.Cu") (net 11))
 (segment (start 89.245 77.307) (end 58.075 77.307) (width 0.25) (layer "F.Cu") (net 11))
 (segment (start 123.698 61.024) (end 123.698 62.563604) (width 0.25) (layer "F.Cu") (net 11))
 (segment (start 123.698 62.563604) (end 126.384743 65.250347) (width 0.25) (layer "F.Cu") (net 11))
 (via (at 89.916 77.978) (size 0.8) (drill 0.4) (layers "F.Cu" "B.Cu") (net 11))
 (via (at 126.773653 65.250347) (size 0.8) (drill 0.4) (layers "F.Cu" "B.Cu") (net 11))
 (segment (start 118.627305 77.978) (end 89.916 77.978) (width 0.25) (layer "B.Cu") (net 11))
 (segment (start 126.773653 69.831652) (end 118.627305 77.978) (width 0.25) (layer "B.Cu") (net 11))
 (segment (start 126.773653 65.250347) (end 126.773653 69.831652) (width 0.25) (layer "B.Cu") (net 11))
 (segment (start 88.229 72.227) (end 58.075 72.227) (width 0.25) (layer "F.Cu") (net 9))
 (segment (start 89.154 73.152) (end 88.229 72.227) (width 0.25) (layer "F.Cu") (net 9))
 (segment (start 115.22 59.594) (end 115.062 59.436) (width 0.25) (layer "F.Cu") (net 9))
 (segment (start 58.075 72.227) (end 57.15 73.152) (width 0.25) (layer "F.Cu") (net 9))
 (segment (start 119.768 59.594) (end 115.22 59.594) (width 0.25) (layer "F.Cu") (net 9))
 (via (at 89.154 73.152) (size 0.8) (drill 0.4) (layers "F.Cu" "B.Cu") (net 9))
 (via (at 115.062 59.436) (size 0.8) (drill 0.4) (layers "F.Cu" "B.Cu") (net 9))
 (segment (start 115.062 64.77) (end 115.337 65.045) (width 0.25) (layer "B.Cu") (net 9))
 (segment (start 124.921695 59.473) (end 125.522305 59.473) (width 0.25) (layer "B.Cu") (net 9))
 (segment (start 115.337 65.045) (end 119.349695 65.045) (width 0.25) (layer "B.Cu") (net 9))
 (segment (start 125.947 62.521) (end 115.316 73.152) (width 0.25) (layer "B.Cu") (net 9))
 (segment (start 115.316 73.152) (end 113.538 73.152) (width 0.25) (layer "B.Cu") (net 9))
 (segment (start 125.947 59.897695) (end 125.947 62.521) (width 0.25) (layer "B.Cu") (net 9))
 (segment (start 115.062 59.436) (end 115.062 64.77) (width 0.25) (layer "B.Cu") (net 9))
 (segment (start 125.522305 59.473) (end 125.947 59.897695) (width 0.25) (layer "B.Cu") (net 9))
 (segment (start 119.349695 65.045) (end 124.921695 59.473) (width 0.25) (layer "B.Cu") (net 9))
 (segment (start 113.538 73.152) (end 89.154 73.152) (width 0.25) (layer "B.Cu") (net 9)))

